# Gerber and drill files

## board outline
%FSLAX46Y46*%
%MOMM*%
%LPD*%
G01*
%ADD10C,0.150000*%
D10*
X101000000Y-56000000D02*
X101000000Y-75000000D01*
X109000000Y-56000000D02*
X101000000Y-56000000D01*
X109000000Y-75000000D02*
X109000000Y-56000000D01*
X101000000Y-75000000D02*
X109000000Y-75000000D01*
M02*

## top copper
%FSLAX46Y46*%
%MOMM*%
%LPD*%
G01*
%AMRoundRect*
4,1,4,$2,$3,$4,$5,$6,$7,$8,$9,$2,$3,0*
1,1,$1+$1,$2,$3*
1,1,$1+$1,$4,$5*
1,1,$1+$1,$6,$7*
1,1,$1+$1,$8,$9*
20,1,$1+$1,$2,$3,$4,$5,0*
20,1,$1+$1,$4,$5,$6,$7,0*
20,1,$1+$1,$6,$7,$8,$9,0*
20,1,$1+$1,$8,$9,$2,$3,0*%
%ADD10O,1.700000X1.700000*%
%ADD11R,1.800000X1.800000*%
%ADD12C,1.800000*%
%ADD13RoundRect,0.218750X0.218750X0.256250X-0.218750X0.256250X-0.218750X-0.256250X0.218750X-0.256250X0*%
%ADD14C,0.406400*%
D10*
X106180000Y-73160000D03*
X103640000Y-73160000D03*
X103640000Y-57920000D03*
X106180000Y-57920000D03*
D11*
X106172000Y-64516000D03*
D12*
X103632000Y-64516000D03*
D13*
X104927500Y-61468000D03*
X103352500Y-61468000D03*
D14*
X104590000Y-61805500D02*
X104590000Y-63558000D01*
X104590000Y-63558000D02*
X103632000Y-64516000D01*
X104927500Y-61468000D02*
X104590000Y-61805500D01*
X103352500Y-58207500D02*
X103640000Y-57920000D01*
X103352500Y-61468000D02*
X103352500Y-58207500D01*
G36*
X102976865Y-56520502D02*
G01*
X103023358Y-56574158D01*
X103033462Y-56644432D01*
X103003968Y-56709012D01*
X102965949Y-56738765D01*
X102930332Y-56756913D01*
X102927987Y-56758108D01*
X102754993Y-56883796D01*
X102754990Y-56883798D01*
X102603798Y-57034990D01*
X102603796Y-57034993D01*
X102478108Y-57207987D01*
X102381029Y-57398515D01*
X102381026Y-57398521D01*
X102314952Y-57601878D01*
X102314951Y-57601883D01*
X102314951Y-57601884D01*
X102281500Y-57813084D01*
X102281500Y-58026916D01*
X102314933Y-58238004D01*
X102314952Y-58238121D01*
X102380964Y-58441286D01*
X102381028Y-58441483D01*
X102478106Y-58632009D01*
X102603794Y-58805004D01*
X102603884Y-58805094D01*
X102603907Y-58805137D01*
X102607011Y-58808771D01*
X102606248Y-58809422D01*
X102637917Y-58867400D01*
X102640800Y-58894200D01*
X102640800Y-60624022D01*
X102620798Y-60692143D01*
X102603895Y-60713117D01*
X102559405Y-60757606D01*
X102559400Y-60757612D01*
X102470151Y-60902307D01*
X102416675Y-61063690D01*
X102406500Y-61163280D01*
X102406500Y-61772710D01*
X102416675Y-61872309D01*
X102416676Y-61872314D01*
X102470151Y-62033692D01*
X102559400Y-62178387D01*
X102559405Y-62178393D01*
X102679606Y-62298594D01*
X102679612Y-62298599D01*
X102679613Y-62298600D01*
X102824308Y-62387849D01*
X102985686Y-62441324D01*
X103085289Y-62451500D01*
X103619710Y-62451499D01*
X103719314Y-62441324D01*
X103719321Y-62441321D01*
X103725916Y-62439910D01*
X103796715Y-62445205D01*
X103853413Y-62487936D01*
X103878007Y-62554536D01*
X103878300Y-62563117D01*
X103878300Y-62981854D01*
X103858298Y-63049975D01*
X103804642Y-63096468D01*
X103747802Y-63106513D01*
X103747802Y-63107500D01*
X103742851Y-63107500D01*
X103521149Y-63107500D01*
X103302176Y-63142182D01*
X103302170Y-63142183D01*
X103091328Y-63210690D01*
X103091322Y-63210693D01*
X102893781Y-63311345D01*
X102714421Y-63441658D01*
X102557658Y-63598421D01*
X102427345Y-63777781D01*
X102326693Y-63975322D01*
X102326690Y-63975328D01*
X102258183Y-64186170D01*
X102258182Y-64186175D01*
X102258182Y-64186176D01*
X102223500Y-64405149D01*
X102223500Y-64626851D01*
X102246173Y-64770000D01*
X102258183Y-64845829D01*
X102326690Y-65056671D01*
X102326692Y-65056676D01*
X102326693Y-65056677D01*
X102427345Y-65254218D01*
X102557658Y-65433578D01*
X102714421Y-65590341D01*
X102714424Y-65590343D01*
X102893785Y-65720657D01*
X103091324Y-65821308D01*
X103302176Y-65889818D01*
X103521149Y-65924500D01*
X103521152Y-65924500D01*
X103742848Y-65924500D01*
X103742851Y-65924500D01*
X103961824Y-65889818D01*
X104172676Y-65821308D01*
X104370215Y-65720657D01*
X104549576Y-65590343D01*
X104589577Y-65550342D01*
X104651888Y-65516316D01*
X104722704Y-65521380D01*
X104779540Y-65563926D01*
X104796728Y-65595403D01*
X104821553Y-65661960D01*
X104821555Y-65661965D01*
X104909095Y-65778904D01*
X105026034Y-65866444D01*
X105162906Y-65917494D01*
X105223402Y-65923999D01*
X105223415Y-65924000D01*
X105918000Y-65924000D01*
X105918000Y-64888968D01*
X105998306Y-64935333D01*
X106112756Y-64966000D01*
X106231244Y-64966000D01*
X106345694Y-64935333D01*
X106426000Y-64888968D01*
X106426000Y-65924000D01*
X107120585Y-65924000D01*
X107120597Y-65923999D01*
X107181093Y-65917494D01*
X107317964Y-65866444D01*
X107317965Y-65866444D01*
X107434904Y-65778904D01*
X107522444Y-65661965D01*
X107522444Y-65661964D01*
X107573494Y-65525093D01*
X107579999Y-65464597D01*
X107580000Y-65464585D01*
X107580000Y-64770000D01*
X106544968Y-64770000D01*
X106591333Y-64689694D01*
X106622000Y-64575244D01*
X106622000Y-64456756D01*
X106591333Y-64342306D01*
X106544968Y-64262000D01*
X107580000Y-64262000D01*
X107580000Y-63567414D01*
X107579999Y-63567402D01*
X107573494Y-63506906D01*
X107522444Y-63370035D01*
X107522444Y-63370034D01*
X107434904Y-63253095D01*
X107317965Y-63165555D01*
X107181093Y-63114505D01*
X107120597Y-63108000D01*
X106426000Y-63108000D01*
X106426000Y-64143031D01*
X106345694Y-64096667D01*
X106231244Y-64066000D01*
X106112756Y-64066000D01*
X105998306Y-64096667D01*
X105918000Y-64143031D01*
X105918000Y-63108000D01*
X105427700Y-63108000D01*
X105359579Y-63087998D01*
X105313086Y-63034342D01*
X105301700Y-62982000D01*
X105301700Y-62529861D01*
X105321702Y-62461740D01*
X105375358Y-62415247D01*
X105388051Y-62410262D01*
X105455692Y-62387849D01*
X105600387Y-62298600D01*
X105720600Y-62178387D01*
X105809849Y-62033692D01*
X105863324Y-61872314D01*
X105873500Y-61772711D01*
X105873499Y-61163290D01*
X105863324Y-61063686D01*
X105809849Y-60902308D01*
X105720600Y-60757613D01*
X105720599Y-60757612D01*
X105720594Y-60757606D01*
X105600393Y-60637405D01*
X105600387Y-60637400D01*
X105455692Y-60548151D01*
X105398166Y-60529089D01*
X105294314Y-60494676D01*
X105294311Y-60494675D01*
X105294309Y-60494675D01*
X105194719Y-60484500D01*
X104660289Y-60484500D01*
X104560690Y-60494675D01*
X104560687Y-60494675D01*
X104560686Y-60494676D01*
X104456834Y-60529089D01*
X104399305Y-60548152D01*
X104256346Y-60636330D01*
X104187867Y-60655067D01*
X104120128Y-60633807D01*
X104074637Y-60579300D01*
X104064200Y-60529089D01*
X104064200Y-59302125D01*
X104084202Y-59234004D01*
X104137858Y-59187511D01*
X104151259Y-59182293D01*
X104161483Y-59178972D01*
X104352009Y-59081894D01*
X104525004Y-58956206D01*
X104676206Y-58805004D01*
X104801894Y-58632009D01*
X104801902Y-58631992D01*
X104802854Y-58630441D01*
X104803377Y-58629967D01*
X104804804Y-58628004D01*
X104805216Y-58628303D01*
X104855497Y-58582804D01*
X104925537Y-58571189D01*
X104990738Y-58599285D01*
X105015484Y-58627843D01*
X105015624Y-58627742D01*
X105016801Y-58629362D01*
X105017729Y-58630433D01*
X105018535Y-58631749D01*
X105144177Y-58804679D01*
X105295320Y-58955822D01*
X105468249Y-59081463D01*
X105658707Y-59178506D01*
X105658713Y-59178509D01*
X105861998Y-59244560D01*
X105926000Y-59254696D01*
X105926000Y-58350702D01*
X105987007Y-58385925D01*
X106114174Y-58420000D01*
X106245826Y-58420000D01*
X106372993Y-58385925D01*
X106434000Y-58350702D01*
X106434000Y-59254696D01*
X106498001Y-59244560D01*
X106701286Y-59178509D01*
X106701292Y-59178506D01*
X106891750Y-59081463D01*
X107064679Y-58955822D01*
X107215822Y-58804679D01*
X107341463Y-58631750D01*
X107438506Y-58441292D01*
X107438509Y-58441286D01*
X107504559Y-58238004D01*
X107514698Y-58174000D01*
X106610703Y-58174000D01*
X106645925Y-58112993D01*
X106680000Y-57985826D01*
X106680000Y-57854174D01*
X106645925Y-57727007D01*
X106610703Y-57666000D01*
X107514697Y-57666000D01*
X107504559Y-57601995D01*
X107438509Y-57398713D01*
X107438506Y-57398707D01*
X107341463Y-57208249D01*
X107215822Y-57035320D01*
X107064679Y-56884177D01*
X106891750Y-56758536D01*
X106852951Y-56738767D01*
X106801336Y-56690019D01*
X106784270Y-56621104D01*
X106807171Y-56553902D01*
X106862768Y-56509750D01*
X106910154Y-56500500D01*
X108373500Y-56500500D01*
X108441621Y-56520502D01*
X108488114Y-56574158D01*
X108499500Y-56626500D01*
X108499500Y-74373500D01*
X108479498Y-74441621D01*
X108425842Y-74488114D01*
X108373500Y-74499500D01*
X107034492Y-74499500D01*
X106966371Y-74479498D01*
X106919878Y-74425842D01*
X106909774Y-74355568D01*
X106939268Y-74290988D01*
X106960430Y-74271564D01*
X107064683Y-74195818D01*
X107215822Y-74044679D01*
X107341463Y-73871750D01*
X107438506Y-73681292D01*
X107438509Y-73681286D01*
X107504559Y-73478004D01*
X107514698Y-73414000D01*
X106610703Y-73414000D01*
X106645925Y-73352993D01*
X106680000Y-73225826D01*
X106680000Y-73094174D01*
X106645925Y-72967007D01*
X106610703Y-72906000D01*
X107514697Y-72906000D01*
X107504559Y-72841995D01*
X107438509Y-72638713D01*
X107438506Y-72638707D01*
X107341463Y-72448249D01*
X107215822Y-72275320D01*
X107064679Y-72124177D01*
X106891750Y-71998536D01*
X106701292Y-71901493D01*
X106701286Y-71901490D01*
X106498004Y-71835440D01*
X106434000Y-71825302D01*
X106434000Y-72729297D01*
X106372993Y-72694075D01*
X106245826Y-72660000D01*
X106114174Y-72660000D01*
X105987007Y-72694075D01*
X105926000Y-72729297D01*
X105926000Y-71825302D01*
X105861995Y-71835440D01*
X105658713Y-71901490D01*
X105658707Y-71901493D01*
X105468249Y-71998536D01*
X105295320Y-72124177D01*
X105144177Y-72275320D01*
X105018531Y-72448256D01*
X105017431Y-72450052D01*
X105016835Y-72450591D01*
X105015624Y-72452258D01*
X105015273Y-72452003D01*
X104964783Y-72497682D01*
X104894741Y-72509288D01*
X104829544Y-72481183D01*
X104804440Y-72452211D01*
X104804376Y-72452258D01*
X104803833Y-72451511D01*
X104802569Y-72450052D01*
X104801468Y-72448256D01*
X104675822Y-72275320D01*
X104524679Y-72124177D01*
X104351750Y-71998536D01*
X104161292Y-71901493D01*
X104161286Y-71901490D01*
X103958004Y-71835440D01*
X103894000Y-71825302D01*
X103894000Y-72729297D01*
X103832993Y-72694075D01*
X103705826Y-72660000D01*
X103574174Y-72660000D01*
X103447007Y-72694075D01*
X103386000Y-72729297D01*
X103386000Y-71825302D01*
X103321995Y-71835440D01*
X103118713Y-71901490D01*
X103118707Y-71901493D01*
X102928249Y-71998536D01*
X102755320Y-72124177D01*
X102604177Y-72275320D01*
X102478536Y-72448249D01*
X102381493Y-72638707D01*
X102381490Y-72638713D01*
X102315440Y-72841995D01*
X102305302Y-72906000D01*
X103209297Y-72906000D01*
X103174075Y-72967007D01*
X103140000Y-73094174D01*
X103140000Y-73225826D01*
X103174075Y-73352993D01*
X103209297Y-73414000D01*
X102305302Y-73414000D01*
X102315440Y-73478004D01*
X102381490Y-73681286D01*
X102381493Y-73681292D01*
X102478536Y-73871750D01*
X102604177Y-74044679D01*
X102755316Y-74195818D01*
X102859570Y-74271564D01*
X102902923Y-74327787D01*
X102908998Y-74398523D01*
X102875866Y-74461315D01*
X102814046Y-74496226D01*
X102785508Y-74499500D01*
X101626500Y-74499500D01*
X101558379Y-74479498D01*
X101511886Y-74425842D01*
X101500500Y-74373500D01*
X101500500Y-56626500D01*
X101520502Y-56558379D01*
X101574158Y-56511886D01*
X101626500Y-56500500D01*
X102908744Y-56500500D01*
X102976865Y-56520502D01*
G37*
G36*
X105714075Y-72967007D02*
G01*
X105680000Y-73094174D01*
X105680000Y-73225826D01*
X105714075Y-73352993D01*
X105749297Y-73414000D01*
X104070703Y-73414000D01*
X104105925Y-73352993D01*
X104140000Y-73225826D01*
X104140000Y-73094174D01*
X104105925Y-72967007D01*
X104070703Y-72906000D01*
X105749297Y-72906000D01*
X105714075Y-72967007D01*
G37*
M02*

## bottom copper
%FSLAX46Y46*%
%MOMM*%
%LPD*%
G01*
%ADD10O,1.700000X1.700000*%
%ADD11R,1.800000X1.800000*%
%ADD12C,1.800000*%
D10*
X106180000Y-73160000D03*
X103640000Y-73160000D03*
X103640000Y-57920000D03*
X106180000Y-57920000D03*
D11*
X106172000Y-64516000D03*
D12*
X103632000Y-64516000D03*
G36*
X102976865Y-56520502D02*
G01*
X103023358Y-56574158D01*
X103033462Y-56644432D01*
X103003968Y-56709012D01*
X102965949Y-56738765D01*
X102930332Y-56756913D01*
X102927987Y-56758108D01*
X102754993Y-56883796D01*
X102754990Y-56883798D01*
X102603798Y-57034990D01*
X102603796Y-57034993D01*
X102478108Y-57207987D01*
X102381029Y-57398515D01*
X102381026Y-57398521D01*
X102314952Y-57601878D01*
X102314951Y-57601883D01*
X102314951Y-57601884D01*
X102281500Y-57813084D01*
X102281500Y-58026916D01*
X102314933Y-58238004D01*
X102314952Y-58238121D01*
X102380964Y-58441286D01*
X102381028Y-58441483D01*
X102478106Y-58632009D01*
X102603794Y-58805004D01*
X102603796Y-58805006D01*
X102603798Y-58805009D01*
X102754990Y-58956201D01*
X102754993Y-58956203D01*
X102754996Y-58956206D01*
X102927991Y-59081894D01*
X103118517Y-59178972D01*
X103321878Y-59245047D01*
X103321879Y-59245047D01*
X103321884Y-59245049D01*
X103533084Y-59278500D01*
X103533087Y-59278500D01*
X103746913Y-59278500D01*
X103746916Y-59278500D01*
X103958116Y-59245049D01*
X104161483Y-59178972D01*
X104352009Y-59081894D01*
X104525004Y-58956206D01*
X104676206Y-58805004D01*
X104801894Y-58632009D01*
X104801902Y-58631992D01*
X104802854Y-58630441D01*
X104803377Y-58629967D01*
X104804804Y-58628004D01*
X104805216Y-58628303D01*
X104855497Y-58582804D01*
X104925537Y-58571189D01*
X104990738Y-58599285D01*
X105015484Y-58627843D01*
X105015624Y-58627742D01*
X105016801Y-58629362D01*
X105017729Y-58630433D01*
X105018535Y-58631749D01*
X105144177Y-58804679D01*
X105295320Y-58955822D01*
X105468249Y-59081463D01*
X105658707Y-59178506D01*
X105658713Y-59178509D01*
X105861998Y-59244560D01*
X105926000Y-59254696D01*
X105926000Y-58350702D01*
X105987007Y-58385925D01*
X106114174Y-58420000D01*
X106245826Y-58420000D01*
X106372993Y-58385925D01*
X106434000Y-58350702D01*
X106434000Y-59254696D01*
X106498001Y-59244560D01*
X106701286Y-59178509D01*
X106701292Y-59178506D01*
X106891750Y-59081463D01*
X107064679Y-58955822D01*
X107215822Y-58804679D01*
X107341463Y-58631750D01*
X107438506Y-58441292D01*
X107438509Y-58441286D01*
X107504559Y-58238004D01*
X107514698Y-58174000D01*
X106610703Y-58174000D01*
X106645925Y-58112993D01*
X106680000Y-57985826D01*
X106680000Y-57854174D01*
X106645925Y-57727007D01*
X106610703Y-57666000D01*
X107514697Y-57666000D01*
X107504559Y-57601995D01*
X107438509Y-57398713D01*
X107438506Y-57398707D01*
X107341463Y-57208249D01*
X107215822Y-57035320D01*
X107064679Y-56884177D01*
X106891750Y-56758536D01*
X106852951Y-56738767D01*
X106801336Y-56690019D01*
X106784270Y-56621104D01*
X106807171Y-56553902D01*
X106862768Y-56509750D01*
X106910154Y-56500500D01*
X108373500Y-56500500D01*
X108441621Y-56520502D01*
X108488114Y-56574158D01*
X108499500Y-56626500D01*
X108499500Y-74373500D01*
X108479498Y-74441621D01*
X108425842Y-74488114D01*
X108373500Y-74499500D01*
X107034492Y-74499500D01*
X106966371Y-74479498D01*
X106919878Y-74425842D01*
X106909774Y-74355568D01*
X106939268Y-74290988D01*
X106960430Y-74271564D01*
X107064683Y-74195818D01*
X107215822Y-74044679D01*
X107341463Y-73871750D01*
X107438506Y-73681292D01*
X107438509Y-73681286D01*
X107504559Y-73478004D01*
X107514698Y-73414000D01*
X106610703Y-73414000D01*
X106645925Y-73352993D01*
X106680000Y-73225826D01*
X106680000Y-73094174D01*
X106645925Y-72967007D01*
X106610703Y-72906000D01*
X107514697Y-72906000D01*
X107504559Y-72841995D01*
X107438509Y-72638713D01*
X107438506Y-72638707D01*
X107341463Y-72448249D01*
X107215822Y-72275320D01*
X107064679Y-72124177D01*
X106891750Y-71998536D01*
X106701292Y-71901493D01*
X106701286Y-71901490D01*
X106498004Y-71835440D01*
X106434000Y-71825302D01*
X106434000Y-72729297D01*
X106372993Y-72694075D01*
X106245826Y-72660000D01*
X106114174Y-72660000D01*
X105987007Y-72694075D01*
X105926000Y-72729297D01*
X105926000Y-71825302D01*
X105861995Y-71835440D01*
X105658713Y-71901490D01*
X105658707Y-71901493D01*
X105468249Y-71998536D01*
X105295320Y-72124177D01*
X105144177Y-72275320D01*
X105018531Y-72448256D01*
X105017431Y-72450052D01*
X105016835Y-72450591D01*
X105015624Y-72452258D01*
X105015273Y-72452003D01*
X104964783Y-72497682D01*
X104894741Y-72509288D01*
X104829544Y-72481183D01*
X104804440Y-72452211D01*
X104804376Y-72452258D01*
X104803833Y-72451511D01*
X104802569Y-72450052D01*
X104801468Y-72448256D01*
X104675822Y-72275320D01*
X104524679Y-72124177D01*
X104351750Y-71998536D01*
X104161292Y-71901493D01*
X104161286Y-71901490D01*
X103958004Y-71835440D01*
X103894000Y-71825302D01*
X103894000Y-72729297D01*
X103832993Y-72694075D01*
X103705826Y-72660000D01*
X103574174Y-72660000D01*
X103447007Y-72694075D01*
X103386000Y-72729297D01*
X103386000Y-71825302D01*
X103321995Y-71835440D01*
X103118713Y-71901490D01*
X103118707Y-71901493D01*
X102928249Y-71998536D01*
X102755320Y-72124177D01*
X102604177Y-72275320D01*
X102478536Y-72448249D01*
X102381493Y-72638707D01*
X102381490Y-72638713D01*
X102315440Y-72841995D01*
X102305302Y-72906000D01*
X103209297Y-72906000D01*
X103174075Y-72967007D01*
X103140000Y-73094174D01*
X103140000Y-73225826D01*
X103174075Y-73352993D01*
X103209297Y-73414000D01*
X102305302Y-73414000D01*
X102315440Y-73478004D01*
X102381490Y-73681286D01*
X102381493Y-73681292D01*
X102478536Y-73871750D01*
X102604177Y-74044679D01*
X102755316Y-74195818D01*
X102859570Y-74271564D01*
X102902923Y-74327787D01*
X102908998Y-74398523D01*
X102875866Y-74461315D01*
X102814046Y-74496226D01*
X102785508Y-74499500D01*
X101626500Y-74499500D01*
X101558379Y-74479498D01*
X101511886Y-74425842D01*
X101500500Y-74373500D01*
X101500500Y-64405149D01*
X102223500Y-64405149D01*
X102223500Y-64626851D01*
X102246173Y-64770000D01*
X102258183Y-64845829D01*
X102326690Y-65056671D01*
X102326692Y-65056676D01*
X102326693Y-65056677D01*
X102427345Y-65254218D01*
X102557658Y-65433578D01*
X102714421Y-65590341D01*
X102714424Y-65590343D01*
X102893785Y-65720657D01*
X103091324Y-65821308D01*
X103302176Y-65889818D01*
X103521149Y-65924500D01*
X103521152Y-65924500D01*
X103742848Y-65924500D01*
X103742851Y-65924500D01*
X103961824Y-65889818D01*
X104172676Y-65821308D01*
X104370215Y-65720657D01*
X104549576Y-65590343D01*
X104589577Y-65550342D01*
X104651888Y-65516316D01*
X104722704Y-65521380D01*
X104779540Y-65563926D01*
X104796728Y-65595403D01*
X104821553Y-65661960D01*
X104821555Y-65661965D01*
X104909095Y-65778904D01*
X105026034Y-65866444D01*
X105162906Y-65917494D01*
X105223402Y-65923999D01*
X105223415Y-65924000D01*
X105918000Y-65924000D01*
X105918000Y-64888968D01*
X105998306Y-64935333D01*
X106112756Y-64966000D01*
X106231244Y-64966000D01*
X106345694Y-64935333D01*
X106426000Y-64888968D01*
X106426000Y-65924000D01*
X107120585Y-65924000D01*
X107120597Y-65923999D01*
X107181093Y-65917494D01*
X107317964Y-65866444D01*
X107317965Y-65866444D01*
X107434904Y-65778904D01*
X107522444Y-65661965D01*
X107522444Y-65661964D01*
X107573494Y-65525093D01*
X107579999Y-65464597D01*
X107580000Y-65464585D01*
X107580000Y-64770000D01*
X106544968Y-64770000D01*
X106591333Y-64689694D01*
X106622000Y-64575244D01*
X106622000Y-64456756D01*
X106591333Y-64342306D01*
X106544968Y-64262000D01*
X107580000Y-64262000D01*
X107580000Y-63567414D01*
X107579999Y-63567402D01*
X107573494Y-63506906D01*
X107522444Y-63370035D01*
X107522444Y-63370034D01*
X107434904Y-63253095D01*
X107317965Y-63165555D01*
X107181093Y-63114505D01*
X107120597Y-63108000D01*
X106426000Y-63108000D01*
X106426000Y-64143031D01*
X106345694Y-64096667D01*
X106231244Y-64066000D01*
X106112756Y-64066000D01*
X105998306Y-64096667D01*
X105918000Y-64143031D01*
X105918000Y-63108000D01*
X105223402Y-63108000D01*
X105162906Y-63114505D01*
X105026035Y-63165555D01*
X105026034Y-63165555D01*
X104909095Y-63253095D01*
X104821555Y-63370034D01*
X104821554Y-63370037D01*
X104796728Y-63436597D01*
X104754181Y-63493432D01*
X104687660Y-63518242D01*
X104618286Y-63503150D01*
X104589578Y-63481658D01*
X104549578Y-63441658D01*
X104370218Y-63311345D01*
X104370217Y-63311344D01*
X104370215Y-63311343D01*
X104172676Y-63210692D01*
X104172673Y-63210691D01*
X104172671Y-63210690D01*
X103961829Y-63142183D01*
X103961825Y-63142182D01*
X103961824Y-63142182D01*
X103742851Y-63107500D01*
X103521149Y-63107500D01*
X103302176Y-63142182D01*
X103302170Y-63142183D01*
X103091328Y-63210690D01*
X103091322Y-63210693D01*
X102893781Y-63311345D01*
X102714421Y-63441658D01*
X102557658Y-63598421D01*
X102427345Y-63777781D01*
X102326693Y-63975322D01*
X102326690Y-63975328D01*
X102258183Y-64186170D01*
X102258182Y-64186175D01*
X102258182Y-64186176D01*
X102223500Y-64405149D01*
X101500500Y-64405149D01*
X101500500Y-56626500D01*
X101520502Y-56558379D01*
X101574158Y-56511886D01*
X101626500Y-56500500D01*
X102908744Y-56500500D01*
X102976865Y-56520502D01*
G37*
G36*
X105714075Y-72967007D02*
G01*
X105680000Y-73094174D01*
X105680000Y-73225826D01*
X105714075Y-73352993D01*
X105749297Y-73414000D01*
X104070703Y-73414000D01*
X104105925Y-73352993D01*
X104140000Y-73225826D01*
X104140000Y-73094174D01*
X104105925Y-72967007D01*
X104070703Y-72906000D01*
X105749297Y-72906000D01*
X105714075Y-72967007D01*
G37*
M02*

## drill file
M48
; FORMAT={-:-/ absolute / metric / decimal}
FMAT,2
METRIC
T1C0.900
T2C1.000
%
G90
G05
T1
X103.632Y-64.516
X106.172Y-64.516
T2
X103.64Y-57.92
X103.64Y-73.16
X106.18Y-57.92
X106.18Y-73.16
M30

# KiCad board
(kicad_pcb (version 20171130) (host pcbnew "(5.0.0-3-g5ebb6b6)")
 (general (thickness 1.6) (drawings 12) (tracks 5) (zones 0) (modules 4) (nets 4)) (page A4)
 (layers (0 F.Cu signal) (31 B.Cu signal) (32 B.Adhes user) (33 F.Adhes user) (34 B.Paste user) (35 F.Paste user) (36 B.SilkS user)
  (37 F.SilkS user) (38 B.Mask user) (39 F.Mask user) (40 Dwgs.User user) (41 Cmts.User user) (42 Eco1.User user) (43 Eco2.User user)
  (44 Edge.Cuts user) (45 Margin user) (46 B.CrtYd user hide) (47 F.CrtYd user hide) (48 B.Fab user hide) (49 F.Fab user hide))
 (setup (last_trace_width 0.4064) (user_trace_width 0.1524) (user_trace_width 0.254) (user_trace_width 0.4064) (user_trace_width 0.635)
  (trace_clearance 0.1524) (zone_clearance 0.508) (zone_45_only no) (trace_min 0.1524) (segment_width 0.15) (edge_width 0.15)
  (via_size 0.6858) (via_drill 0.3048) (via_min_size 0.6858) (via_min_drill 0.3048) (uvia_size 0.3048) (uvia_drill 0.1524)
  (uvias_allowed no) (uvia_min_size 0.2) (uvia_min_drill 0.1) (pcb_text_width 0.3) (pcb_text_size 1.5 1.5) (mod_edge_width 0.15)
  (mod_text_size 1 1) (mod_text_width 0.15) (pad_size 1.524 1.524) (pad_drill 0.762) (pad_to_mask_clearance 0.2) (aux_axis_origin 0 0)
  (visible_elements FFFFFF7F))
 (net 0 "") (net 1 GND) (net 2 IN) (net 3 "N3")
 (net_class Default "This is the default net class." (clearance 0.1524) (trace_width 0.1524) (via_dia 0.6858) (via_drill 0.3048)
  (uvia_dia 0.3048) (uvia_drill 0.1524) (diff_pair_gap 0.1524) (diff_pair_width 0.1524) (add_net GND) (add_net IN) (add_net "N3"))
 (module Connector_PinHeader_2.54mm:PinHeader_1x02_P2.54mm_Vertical (layer B.Cu) (at 103.64 73.16 270)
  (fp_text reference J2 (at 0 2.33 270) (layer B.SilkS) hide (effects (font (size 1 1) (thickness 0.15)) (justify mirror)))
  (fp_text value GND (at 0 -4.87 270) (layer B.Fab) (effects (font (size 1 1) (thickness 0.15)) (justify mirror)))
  (pad 2 thru_hole oval (at 0 -2.54 270) (size 1.7 1.7) (drill 1) (layers *.Cu *.Mask) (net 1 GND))
  (pad 1 thru_hole oval (at 0 0 270) (size 1.7 1.7) (drill 1) (layers *.Cu *.Mask) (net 1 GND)))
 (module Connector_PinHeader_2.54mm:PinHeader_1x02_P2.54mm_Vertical (layer B.Cu) (at 103.64 57.92 270)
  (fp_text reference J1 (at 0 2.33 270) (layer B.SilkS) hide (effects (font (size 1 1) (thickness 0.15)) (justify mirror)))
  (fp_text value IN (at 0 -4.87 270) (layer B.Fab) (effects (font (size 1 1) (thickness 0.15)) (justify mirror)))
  (pad 1 thru_hole oval (at 0 0 270) (size 1.7 1.7) (drill 1) (layers *.Cu *.Mask) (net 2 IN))
  (pad 2 thru_hole oval (at 0 -2.54 270) (size 1.7 1.7) (drill 1) (layers *.Cu *.Mask) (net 1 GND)))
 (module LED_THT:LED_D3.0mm (layer F.Cu) (at 106.172 64.516 180)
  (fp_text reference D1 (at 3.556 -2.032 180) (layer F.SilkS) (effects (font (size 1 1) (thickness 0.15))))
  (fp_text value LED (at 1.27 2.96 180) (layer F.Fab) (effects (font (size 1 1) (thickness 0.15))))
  (pad 1 thru_hole rect (at 0 0 180) (size 1.8 1.8) (drill 0.9) (layers *.Cu *.Mask) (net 1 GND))
  (pad 2 thru_hole circle (at 2.54 0 180) (size 1.8 1.8) (drill 0.9) (layers *.Cu *.Mask) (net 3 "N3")))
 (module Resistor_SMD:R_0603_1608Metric (layer F.Cu) (at 104.14 61.468 180)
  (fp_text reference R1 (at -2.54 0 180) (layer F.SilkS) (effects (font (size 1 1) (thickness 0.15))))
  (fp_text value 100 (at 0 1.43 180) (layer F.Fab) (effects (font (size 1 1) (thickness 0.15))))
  (pad 1 smd roundrect (at -0.7875 0 180) (size 0.875 0.95) (layers F.Cu F.Paste F.Mask) (roundrect_rratio 0.25) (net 3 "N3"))
  (pad 2 smd roundrect (at 0.7875 0 180) (size 0.875 0.95) (layers F.Cu F.Paste F.Mask) (roundrect_rratio 0.25) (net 2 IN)))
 (gr_line (start 101 56) (end 101 75) (layer Edge.Cuts) (width 0.15))
 (gr_line (start 109 56) (end 101 56) (layer Edge.Cuts) (width 0.15))
 (gr_line (start 109 75) (end 109 56) (layer Edge.Cuts) (width 0.15))
 (gr_line (start 101 75) (end 109 75) (layer Edge.Cuts) (width 0.15))
 (segment (start 104.59 61.8055) (end 104.59 63.558) (width 0.4064) (layer F.Cu) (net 3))
 (segment (start 104.59 63.558) (end 103.632 64.516) (width 0.4064) (layer F.Cu) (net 3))
 (segment (start 104.9275 61.468) (end 104.59 61.8055) (width 0.4064) (layer F.Cu) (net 3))
 (segment (start 103.3525 58.2075) (end 103.64 57.92) (width 0.4064) (layer F.Cu) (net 2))
 (segment (start 103.3525 61.468) (end 103.3525 58.2075) (width 0.4064) (layer F.Cu) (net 2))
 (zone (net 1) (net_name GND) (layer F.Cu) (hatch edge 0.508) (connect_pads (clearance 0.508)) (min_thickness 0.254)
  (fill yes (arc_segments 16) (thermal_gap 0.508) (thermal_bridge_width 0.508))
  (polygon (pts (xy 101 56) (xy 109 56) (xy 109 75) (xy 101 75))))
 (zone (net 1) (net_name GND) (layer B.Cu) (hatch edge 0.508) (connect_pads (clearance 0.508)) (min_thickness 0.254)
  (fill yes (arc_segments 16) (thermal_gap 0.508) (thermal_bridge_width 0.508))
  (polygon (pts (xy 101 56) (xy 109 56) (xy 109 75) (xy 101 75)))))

